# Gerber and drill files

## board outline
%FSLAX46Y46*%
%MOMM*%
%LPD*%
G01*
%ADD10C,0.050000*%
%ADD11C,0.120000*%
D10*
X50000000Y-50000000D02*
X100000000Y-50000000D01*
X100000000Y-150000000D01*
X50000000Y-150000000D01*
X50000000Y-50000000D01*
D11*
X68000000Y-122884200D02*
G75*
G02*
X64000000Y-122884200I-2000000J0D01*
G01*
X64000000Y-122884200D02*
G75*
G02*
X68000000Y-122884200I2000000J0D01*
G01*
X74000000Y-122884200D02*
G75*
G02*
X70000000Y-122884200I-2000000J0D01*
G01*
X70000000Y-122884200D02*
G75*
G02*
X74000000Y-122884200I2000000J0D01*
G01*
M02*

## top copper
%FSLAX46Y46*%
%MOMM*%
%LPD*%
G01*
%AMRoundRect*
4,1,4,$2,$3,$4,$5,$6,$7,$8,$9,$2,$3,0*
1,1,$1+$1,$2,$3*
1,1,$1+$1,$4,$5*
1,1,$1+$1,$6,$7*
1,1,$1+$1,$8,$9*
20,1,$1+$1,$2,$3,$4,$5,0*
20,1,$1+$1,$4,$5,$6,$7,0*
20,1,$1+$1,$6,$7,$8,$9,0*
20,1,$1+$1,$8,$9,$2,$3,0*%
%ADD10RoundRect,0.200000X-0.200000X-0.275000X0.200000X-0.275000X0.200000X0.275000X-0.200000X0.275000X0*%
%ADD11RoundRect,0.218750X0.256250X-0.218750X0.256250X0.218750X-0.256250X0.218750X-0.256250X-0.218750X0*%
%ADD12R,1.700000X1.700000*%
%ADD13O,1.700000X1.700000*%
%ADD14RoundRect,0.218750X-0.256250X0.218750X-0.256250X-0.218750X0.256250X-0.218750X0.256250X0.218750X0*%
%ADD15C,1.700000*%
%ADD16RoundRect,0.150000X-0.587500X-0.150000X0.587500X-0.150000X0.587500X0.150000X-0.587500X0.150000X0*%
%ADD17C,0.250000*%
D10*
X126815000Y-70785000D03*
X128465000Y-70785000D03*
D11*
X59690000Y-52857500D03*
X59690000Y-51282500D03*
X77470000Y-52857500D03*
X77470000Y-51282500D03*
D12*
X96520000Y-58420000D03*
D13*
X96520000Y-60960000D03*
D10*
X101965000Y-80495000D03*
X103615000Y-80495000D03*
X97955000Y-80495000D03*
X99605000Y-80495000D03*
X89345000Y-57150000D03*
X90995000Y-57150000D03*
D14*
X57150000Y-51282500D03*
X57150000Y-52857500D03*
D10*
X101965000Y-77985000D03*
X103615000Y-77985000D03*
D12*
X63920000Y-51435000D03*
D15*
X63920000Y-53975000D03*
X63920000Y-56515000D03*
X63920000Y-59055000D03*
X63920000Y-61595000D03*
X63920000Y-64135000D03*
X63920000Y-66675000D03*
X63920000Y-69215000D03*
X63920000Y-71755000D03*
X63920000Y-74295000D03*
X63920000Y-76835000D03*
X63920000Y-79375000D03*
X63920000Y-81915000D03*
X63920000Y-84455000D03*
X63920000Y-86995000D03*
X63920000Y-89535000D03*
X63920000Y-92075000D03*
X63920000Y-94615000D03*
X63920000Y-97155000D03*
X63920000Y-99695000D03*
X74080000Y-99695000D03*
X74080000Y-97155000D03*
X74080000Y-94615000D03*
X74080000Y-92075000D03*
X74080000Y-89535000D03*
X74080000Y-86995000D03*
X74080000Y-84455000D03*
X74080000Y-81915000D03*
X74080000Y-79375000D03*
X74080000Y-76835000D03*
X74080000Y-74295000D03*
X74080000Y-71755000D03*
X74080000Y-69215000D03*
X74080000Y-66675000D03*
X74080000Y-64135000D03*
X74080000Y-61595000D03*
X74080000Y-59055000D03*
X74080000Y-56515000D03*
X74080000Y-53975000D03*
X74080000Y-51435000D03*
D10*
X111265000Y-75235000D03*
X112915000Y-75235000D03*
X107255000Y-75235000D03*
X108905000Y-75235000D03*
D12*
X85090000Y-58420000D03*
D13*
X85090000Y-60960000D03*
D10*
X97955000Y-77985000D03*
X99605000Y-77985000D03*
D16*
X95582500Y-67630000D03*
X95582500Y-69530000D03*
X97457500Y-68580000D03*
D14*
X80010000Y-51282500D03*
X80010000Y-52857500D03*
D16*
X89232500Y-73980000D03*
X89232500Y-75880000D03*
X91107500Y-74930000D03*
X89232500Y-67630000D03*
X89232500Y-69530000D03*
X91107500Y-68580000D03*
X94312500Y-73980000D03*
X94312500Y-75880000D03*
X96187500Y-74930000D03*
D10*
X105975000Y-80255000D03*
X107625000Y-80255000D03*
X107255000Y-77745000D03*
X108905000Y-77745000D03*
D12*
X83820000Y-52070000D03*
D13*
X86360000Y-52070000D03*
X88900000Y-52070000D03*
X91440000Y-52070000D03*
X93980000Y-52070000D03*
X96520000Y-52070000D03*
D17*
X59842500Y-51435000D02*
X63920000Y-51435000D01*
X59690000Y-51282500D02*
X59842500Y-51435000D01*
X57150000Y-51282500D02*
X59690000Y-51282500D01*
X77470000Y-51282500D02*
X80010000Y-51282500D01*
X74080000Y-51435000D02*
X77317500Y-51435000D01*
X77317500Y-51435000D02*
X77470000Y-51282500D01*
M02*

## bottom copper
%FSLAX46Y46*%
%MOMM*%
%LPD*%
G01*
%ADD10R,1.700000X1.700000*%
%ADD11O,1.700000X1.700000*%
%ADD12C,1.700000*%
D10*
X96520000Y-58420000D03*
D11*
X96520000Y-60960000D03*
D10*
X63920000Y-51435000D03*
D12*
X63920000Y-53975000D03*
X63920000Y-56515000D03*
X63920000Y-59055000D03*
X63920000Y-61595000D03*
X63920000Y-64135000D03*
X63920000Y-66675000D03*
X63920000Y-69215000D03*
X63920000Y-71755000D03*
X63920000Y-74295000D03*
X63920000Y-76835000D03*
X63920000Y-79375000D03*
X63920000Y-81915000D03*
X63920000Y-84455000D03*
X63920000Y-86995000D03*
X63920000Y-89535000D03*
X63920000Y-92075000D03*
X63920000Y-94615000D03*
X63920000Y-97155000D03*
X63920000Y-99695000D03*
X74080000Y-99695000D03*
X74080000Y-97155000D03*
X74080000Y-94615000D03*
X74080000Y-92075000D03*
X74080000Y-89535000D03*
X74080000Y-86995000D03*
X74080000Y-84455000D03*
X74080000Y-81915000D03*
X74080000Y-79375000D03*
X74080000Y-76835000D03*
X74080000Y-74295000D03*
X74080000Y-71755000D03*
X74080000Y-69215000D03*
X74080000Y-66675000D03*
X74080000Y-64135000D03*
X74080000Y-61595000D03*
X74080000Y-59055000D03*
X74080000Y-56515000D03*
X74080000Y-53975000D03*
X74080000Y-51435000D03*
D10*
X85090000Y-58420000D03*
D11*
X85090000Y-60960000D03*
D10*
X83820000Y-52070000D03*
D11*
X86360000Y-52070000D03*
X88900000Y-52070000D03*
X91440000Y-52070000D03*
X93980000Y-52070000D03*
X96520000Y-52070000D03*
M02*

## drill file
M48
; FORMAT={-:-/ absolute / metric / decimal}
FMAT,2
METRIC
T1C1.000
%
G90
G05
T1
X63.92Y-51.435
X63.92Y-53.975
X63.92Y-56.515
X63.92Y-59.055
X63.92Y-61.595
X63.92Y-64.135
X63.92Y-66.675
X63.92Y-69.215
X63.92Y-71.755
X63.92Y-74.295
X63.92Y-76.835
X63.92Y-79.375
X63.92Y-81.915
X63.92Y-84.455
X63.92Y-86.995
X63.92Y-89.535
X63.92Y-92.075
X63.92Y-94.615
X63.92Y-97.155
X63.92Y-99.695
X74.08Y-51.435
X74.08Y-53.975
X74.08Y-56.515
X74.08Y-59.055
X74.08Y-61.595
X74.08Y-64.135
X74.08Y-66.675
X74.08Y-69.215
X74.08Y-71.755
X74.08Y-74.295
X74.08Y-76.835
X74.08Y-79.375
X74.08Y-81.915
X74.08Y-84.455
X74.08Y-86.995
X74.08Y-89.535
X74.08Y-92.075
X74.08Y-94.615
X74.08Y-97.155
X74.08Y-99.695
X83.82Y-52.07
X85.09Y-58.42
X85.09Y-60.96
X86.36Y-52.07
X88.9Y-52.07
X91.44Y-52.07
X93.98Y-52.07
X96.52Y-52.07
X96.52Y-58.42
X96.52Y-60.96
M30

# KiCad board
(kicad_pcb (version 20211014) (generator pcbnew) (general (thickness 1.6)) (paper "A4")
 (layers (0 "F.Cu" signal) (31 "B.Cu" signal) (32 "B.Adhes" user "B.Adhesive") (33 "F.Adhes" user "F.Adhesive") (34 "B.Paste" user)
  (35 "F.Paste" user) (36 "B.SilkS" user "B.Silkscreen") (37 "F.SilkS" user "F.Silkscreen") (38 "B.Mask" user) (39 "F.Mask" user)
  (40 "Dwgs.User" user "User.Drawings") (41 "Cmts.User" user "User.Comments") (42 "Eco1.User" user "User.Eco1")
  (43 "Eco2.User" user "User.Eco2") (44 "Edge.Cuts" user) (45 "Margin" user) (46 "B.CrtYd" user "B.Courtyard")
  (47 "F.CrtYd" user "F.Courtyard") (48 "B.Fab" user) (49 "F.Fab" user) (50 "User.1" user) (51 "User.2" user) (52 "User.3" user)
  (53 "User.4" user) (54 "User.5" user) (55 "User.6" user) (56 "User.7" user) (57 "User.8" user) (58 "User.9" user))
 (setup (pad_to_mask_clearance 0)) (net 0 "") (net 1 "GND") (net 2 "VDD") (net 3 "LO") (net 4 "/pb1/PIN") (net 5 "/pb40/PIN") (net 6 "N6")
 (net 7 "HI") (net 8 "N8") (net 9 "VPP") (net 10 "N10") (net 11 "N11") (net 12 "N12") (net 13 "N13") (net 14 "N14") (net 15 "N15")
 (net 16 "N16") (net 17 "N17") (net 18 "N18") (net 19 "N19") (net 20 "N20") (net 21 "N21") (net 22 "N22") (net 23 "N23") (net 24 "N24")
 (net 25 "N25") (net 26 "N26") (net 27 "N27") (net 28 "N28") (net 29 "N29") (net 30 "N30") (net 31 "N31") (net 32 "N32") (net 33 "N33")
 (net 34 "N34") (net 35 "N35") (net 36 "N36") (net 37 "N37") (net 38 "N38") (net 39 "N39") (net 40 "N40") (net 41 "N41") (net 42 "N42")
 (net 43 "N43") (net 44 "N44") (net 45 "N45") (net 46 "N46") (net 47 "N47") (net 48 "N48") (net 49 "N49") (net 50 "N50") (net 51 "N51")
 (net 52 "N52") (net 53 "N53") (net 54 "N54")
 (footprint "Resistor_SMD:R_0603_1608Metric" (layer "F.Cu") (at 127.64 70.785)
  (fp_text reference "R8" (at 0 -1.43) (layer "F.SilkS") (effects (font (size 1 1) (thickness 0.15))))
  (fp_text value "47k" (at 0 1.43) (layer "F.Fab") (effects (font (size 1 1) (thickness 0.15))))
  (pad "1" smd roundrect (at -0.825 0) (size 0.8 0.95) (layers "F.Cu" "F.Paste" "F.Mask") (roundrect_rratio 0.25) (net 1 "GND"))
  (pad "2" smd roundrect (at 0.825 0) (size 0.8 0.95) (layers "F.Cu" "F.Paste" "F.Mask") (roundrect_rratio 0.25) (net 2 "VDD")))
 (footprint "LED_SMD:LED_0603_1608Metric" (layer "F.Cu") (at 59.69 52.07 90)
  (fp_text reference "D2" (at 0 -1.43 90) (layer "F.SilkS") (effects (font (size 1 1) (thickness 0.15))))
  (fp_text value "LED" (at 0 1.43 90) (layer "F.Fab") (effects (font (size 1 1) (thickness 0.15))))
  (pad "1" smd roundrect (at -0.7875 0 90) (size 0.875 0.95) (layers "F.Cu" "F.Paste" "F.Mask") (roundrect_rratio 0.25) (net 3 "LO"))
  (pad "2" smd roundrect (at 0.7875 0 90) (size 0.875 0.95) (layers "F.Cu" "F.Paste" "F.Mask") (roundrect_rratio 0.25) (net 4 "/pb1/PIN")))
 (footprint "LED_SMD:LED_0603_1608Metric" (layer "F.Cu") (at 77.47 52.07 90)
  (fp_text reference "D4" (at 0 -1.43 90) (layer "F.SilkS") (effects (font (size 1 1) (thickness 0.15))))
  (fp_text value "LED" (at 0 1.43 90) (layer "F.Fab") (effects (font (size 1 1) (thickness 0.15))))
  (pad "1" smd roundrect (at -0.7875 0 90) (size 0.875 0.95) (layers "F.Cu" "F.Paste" "F.Mask") (roundrect_rratio 0.25) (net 3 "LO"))
  (pad "2" smd roundrect (at 0.7875 0 90) (size 0.875 0.95) (layers "F.Cu" "F.Paste" "F.Mask") (roundrect_rratio 0.25) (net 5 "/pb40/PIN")))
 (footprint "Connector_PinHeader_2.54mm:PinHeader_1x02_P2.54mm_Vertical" (layer "F.Cu") (at 96.52 58.42)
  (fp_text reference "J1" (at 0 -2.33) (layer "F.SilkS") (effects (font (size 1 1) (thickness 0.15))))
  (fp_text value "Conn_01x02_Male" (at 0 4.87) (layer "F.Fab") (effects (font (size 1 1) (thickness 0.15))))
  (pad "1" thru_hole rect (at 0 0) (size 1.7 1.7) (drill 1) (layers *.Cu *.Mask) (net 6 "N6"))
  (pad "2" thru_hole oval (at 0 2.54) (size 1.7 1.7) (drill 1) (layers *.Cu *.Mask) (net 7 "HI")))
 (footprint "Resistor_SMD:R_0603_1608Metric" (layer "F.Cu") (at 102.79 80.495)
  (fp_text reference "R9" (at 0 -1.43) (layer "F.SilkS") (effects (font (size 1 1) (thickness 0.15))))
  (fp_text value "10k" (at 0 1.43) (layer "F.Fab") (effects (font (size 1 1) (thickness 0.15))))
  (pad "1" smd roundrect (at -0.825 0) (size 0.8 0.95) (layers "F.Cu" "F.Paste" "F.Mask") (roundrect_rratio 0.25) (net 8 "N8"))
  (pad "2" smd roundrect (at 0.825 0) (size 0.8 0.95) (layers "F.Cu" "F.Paste" "F.Mask") (roundrect_rratio 0.25) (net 3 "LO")))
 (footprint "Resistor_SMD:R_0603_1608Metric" (layer "F.Cu") (at 98.78 80.495)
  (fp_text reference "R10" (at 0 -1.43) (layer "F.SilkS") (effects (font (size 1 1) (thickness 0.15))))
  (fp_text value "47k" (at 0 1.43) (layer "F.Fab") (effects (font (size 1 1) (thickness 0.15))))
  (pad "1" smd roundrect (at -0.825 0) (size 0.8 0.95) (layers "F.Cu" "F.Paste" "F.Mask") (roundrect_rratio 0.25) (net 1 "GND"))
  (pad "2" smd roundrect (at 0.825 0) (size 0.8 0.95) (layers "F.Cu" "F.Paste" "F.Mask") (roundrect_rratio 0.25) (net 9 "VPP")))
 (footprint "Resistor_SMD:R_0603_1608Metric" (layer "F.Cu") (at 90.17 57.15)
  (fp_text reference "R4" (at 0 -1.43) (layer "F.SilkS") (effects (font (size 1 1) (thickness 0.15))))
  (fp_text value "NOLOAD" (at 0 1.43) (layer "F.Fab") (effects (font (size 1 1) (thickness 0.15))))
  (pad "1" smd roundrect (at -0.825 0) (size 0.8 0.95) (layers "F.Cu" "F.Paste" "F.Mask") (roundrect_rratio 0.25) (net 1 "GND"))
  (pad "2" smd roundrect (at 0.825 0) (size 0.8 0.95) (layers "F.Cu" "F.Paste" "F.Mask") (roundrect_rratio 0.25) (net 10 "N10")))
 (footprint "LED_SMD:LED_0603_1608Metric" (layer "F.Cu") (at 57.15 52.07 -90)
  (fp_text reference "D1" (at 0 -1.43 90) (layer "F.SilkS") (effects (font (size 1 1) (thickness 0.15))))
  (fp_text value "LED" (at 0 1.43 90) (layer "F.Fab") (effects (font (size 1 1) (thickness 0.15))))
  (pad "1" smd roundrect (at -0.7875 0 270) (size 0.875 0.95) (layers "F.Cu" "F.Paste" "F.Mask") (roundrect_rratio 0.25) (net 4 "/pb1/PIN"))
  (pad "2" smd roundrect (at 0.7875 0 270) (size 0.875 0.95) (layers "F.Cu" "F.Paste" "F.Mask") (roundrect_rratio 0.25) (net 7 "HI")))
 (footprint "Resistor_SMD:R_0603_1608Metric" (layer "F.Cu") (at 102.79 77.985)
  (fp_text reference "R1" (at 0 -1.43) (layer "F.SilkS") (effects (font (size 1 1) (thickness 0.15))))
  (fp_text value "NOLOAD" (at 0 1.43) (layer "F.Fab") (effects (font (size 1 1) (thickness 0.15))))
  (pad "1" smd roundrect (at -0.825 0) (size 0.8 0.95) (layers "F.Cu" "F.Paste" "F.Mask") (roundrect_rratio 0.25) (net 6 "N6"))
  (pad "2" smd roundrect (at 0.825 0) (size 0.8 0.95) (layers "F.Cu" "F.Paste" "F.Mask") (roundrect_rratio 0.25) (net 7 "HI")))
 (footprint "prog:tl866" (layer "F.Cu") (at 69 51.435)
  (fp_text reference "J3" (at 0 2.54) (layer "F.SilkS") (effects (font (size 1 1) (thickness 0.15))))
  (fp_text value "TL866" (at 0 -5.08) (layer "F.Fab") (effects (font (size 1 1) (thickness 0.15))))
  (fp_circle (center -3 71.4492) (end -1 71.4492) (layer "Edge.Cuts") (width 0.12) (fill none))
  (fp_circle (center 3 71.4492) (end 5 71.4492) (layer "Edge.Cuts") (width 0.12) (fill none))
  (pad "1" thru_hole rect (at -5.08 0) (size 1.7 1.7) (drill 1) (layers *.Cu *.Mask) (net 4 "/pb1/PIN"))
  (pad "2" thru_hole circle (at -5.08 2.54) (size 1.7 1.7) (drill 1) (layers *.Cu *.Mask) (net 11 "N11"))
  (pad "3" thru_hole circle (at -5.08 5.08) (size 1.7 1.7) (drill 1) (layers *.Cu *.Mask) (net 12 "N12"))
  (pad "4" thru_hole circle (at -5.08 7.62) (size 1.7 1.7) (drill 1) (layers *.Cu *.Mask) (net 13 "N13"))
  (pad "5" thru_hole circle (at -5.08 10.16) (size 1.7 1.7) (drill 1) (layers *.Cu *.Mask) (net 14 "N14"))
  (pad "6" thru_hole circle (at -5.08 12.7) (size 1.7 1.7) (drill 1) (layers *.Cu *.Mask) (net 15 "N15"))
  (pad "7" thru_hole circle (at -5.08 15.24) (size 1.7 1.7) (drill 1) (layers *.Cu *.Mask) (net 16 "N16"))
  (pad "8" thru_hole circle (at -5.08 17.78) (size 1.7 1.7) (drill 1) (layers *.Cu *.Mask) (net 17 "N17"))
  (pad "9" thru_hole circle (at -5.08 20.32) (size 1.7 1.7) (drill 1) (layers *.Cu *.Mask) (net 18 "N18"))
  (pad "10" thru_hole circle (at -5.08 22.86) (size 1.7 1.7) (drill 1) (layers *.Cu *.Mask) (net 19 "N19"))
  (pad "11" thru_hole circle (at -5.08 25.4) (size 1.7 1.7) (drill 1) (layers *.Cu *.Mask) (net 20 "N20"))
  (pad "12" thru_hole circle (at -5.08 27.94) (size 1.7 1.7) (drill 1) (layers *.Cu *.Mask) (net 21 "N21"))
  (pad "13" thru_hole circle (at -5.08 30.48) (size 1.7 1.7) (drill 1) (layers *.Cu *.Mask) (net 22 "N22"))
  (pad "14" thru_hole circle (at -5.08 33.02) (size 1.7 1.7) (drill 1) (layers *.Cu *.Mask) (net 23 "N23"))
  (pad "15" thru_hole circle (at -5.08 35.56) (size 1.7 1.7) (drill 1) (layers *.Cu *.Mask) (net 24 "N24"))
  (pad "16" thru_hole circle (at -5.08 38.1) (size 1.7 1.7) (drill 1) (layers *.Cu *.Mask) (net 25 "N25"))
  (pad "17" thru_hole circle (at -5.08 40.64) (size 1.7 1.7) (drill 1) (layers *.Cu *.Mask) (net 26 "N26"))
  (pad "18" thru_hole circle (at -5.08 43.18) (size 1.7 1.7) (drill 1) (layers *.Cu *.Mask) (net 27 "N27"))
  (pad "19" thru_hole circle (at -5.08 45.72) (size 1.7 1.7) (drill 1) (layers *.Cu *.Mask) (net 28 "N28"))
  (pad "20" thru_hole circle (at -5.08 48.26) (size 1.7 1.7) (drill 1) (layers *.Cu *.Mask) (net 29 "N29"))
  (pad "21" thru_hole circle (at 5.08 48.26) (size 1.7 1.7) (drill 1) (layers *.Cu *.Mask) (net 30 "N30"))
  (pad "22" thru_hole circle (at 5.08 45.72) (size 1.7 1.7) (drill 1) (layers *.Cu *.Mask) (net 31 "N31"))
  (pad "23" thru_hole circle (at 5.08 43.18) (size 1.7 1.7) (drill 1) (layers *.Cu *.Mask) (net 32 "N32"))
  (pad "24" thru_hole circle (at 5.08 40.64) (size 1.7 1.7) (drill 1) (layers *.Cu *.Mask) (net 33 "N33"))
  (pad "25" thru_hole circle (at 5.08 38.1) (size 1.7 1.7) (drill 1) (layers *.Cu *.Mask) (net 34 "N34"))
  (pad "26" thru_hole circle (at 5.08 35.56) (size 1.7 1.7) (drill 1) (layers *.Cu *.Mask) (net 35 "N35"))
  (pad "27" thru_hole circle (at 5.08 33.02) (size 1.7 1.7) (drill 1) (layers *.Cu *.Mask) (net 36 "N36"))
  (pad "28" thru_hole circle (at 5.08 30.48) (size 1.7 1.7) (drill 1) (layers *.Cu *.Mask) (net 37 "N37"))
  (pad "29" thru_hole circle (at 5.08 27.94) (size 1.7 1.7) (drill 1) (layers *.Cu *.Mask) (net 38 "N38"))
  (pad "30" thru_hole circle (at 5.08 25.4) (size 1.7 1.7) (drill 1) (layers *.Cu *.Mask) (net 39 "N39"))
  (pad "31" thru_hole circle (at 5.08 22.86) (size 1.7 1.7) (drill 1) (layers *.Cu *.Mask) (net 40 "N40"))
  (pad "32" thru_hole circle (at 5.08 20.32) (size 1.7 1.7) (drill 1) (layers *.Cu *.Mask) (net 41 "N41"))
  (pad "33" thru_hole circle (at 5.08 17.78) (size 1.7 1.7) (drill 1) (layers *.Cu *.Mask) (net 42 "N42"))
  (pad "34" thru_hole circle (at 5.08 15.24) (size 1.7 1.7) (drill 1) (layers *.Cu *.Mask) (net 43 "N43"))
  (pad "35" thru_hole circle (at 5.08 12.7) (size 1.7 1.7) (drill 1) (layers *.Cu *.Mask) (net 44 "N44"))
  (pad "36" thru_hole circle (at 5.08 10.16) (size 1.7 1.7) (drill 1) (layers *.Cu *.Mask) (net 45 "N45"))
  (pad "37" thru_hole circle (at 5.08 7.62) (size 1.7 1.7) (drill 1) (layers *.Cu *.Mask) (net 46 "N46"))
  (pad "38" thru_hole circle (at 5.08 5.08) (size 1.7 1.7) (drill 1) (layers *.Cu *.Mask) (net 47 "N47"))
  (pad "39" thru_hole circle (at 5.08 2.54) (size 1.7 1.7) (drill 1) (layers *.Cu *.Mask) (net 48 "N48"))
  (pad "40" thru_hole circle (at 5.08 0) (size 1.7 1.7) (drill 1) (layers *.Cu *.Mask) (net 5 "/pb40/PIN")))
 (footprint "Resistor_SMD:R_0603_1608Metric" (layer "F.Cu") (at 112.09 75.235)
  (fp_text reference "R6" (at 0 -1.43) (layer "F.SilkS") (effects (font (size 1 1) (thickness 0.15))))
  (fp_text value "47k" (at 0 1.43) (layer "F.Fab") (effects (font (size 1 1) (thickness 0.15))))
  (pad "1" smd roundrect (at -0.825 0) (size 0.8 0.95) (layers "F.Cu" "F.Paste" "F.Mask") (roundrect_rratio 0.25) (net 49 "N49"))
  (pad "2" smd roundrect (at 0.825 0) (size 0.8 0.95) (layers "F.Cu" "F.Paste" "F.Mask") (roundrect_rratio 0.25) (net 2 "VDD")))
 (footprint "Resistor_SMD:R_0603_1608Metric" (layer "F.Cu") (at 108.08 75.235)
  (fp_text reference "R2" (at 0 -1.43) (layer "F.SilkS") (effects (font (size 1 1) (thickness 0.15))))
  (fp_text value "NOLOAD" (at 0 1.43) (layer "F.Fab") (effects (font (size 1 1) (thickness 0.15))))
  (pad "1" smd roundrect (at -0.825 0) (size 0.8 0.95) (layers "F.Cu" "F.Paste" "F.Mask") (roundrect_rratio 0.25) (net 2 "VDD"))
  (pad "2" smd roundrect (at 0.825 0) (size 0.8 0.95) (layers "F.Cu" "F.Paste" "F.Mask") (roundrect_rratio 0.25) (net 6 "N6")))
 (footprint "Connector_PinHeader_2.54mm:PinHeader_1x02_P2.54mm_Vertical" (layer "F.Cu") (at 85.09 58.42)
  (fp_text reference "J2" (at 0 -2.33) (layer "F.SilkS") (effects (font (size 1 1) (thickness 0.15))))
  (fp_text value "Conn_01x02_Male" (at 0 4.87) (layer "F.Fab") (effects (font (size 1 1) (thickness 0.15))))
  (pad "1" thru_hole rect (at 0 0) (size 1.7 1.7) (drill 1) (layers *.Cu *.Mask) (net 10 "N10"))
  (pad "2" thru_hole oval (at 0 2.54) (size 1.7 1.7) (drill 1) (layers *.Cu *.Mask) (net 3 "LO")))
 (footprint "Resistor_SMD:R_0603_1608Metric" (layer "F.Cu") (at 98.78 77.985)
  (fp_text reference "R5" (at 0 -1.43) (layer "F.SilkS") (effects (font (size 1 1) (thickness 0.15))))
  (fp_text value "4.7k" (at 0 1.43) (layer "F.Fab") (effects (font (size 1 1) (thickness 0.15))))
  (pad "1" smd roundrect (at -0.825 0) (size 0.8 0.95) (layers "F.Cu" "F.Paste" "F.Mask") (roundrect_rratio 0.25) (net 7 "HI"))
  (pad "2" smd roundrect (at 0.825 0) (size 0.8 0.95) (layers "F.Cu" "F.Paste" "F.Mask") (roundrect_rratio 0.25) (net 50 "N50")))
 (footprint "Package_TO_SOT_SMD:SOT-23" (layer "F.Cu") (at 96.52 68.58)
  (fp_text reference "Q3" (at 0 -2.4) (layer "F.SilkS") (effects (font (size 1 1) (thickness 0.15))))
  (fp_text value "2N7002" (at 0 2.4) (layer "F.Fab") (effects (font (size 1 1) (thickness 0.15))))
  (pad "1" smd roundrect (at -0.9375 -0.95) (size 1.475 0.6) (layers "F.Cu" "F.Paste" "F.Mask") (roundrect_rratio 0.25) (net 2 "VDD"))
  (pad "2" smd roundrect (at -0.9375 0.95) (size 1.475 0.6) (layers "F.Cu" "F.Paste" "F.Mask") (roundrect_rratio 0.25) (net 1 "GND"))
  (pad "3" smd roundrect (at 0.9375 0) (size 1.475 0.6) (layers "F.Cu" "F.Paste" "F.Mask") (roundrect_rratio 0.25) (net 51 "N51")))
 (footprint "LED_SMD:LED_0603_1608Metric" (layer "F.Cu") (at 80.01 52.07 -90)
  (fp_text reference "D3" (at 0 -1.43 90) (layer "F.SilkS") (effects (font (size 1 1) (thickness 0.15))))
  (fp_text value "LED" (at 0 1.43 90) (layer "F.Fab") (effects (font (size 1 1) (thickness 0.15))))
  (pad "1" smd roundrect (at -0.7875 0 270) (size 0.875 0.95) (layers "F.Cu" "F.Paste" "F.Mask") (roundrect_rratio 0.25) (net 5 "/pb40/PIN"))
  (pad "2" smd roundrect (at 0.7875 0 270) (size 0.875 0.95) (layers "F.Cu" "F.Paste" "F.Mask") (roundrect_rratio 0.25) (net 7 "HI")))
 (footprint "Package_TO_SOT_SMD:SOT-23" (layer "F.Cu") (at 90.17 74.93)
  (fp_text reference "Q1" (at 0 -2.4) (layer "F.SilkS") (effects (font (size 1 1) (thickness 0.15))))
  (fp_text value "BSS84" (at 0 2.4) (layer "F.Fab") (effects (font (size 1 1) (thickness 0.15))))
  (pad "1" smd roundrect (at -0.9375 -0.95) (size 1.475 0.6) (layers "F.Cu" "F.Paste" "F.Mask") (roundrect_rratio 0.25) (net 49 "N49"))
  (pad "2" smd roundrect (at -0.9375 0.95) (size 1.475 0.6) (layers "F.Cu" "F.Paste" "F.Mask") (roundrect_rratio 0.25) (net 2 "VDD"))
  (pad "3" smd roundrect (at 0.9375 0) (size 1.475 0.6) (layers "F.Cu" "F.Paste" "F.Mask") (roundrect_rratio 0.25) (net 50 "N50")))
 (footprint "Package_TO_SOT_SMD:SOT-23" (layer "F.Cu") (at 90.17 68.58)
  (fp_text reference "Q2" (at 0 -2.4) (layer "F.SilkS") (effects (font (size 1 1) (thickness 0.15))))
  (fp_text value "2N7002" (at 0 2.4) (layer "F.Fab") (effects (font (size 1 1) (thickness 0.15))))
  (pad "1" smd roundrect (at -0.9375 -0.95) (size 1.475 0.6) (layers "F.Cu" "F.Paste" "F.Mask") (roundrect_rratio 0.25) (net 9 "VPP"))
  (pad "2" smd roundrect (at -0.9375 0.95) (size 1.475 0.6) (layers "F.Cu" "F.Paste" "F.Mask") (roundrect_rratio 0.25) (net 1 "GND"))
  (pad "3" smd roundrect (at 0.9375 0) (size 1.475 0.6) (layers "F.Cu" "F.Paste" "F.Mask") (roundrect_rratio 0.25) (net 49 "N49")))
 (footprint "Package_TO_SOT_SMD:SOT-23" (layer "F.Cu") (at 95.25 74.93)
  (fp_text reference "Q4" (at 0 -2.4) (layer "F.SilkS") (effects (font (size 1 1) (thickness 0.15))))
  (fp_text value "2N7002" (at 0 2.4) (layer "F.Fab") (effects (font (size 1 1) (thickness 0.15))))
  (pad "1" smd roundrect (at -0.9375 -0.95) (size 1.475 0.6) (layers "F.Cu" "F.Paste" "F.Mask") (roundrect_rratio 0.25) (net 9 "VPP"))
  (pad "2" smd roundrect (at -0.9375 0.95) (size 1.475 0.6) (layers "F.Cu" "F.Paste" "F.Mask") (roundrect_rratio 0.25) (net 1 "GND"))
  (pad "3" smd roundrect (at 0.9375 0) (size 1.475 0.6) (layers "F.Cu" "F.Paste" "F.Mask") (roundrect_rratio 0.25) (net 8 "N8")))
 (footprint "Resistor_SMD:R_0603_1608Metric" (layer "F.Cu") (at 106.8 80.255)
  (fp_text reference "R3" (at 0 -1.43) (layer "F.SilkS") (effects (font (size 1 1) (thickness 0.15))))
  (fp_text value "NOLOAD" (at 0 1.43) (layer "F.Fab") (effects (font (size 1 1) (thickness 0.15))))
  (pad "1" smd roundrect (at -0.825 0) (size 0.8 0.95) (layers "F.Cu" "F.Paste" "F.Mask") (roundrect_rratio 0.25) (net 10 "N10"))
  (pad "2" smd roundrect (at 0.825 0) (size 0.8 0.95) (layers "F.Cu" "F.Paste" "F.Mask") (roundrect_rratio 0.25) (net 3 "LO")))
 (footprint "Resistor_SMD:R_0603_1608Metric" (layer "F.Cu") (at 108.08 77.745)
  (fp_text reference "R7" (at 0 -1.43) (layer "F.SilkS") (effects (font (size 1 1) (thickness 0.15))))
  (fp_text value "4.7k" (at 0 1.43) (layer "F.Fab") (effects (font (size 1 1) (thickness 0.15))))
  (pad "1" smd roundrect (at -0.825 0) (size 0.8 0.95) (layers "F.Cu" "F.Paste" "F.Mask") (roundrect_rratio 0.25) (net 51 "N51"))
  (pad "2" smd roundrect (at 0.825 0) (size 0.8 0.95) (layers "F.Cu" "F.Paste" "F.Mask") (roundrect_rratio 0.25) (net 3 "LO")))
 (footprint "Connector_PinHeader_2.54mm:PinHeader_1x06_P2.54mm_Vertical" (layer "F.Cu") (at 83.82 52.07 90)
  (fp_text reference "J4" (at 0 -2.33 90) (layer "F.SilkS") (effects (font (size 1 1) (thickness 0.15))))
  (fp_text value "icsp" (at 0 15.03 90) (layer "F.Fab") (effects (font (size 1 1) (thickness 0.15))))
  (pad "1" thru_hole rect (at 0 0 90) (size 1.7 1.7) (drill 1) (layers *.Cu *.Mask) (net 9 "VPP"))
  (pad "2" thru_hole oval (at 0 2.54 90) (size 1.7 1.7) (drill 1) (layers *.Cu *.Mask) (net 2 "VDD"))
  (pad "3" thru_hole oval (at 0 5.08 90) (size 1.7 1.7) (drill 1) (layers *.Cu *.Mask) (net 1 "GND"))
  (pad "4" thru_hole oval (at 0 7.62 90) (size 1.7 1.7) (drill 1) (layers *.Cu *.Mask) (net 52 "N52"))
  (pad "5" thru_hole oval (at 0 10.16 90) (size 1.7 1.7) (drill 1) (layers *.Cu *.Mask) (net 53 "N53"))
  (pad "6" thru_hole oval (at 0 12.7 90) (size 1.7 1.7) (drill 1) (layers *.Cu *.Mask) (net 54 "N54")))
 (gr_rect locked (start 50 50) (end 100 150) (layer "Edge.Cuts") (width 0.05) (fill none))
 (segment (start 59.8425 51.435) (end 63.92 51.435) (width 0.25) (layer "F.Cu") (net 4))
 (segment (start 59.69 51.2825) (end 59.8425 51.435) (width 0.25) (layer "F.Cu") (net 4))
 (segment (start 57.15 51.2825) (end 59.69 51.2825) (width 0.25) (layer "F.Cu") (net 4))
 (segment (start 77.47 51.2825) (end 80.01 51.2825) (width 0.25) (layer "F.Cu") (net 5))
 (segment (start 74.08 51.435) (end 77.3175 51.435) (width 0.25) (layer "F.Cu") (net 5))
 (segment (start 77.3175 51.435) (end 77.47 51.2825) (width 0.25) (layer "F.Cu") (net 5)))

